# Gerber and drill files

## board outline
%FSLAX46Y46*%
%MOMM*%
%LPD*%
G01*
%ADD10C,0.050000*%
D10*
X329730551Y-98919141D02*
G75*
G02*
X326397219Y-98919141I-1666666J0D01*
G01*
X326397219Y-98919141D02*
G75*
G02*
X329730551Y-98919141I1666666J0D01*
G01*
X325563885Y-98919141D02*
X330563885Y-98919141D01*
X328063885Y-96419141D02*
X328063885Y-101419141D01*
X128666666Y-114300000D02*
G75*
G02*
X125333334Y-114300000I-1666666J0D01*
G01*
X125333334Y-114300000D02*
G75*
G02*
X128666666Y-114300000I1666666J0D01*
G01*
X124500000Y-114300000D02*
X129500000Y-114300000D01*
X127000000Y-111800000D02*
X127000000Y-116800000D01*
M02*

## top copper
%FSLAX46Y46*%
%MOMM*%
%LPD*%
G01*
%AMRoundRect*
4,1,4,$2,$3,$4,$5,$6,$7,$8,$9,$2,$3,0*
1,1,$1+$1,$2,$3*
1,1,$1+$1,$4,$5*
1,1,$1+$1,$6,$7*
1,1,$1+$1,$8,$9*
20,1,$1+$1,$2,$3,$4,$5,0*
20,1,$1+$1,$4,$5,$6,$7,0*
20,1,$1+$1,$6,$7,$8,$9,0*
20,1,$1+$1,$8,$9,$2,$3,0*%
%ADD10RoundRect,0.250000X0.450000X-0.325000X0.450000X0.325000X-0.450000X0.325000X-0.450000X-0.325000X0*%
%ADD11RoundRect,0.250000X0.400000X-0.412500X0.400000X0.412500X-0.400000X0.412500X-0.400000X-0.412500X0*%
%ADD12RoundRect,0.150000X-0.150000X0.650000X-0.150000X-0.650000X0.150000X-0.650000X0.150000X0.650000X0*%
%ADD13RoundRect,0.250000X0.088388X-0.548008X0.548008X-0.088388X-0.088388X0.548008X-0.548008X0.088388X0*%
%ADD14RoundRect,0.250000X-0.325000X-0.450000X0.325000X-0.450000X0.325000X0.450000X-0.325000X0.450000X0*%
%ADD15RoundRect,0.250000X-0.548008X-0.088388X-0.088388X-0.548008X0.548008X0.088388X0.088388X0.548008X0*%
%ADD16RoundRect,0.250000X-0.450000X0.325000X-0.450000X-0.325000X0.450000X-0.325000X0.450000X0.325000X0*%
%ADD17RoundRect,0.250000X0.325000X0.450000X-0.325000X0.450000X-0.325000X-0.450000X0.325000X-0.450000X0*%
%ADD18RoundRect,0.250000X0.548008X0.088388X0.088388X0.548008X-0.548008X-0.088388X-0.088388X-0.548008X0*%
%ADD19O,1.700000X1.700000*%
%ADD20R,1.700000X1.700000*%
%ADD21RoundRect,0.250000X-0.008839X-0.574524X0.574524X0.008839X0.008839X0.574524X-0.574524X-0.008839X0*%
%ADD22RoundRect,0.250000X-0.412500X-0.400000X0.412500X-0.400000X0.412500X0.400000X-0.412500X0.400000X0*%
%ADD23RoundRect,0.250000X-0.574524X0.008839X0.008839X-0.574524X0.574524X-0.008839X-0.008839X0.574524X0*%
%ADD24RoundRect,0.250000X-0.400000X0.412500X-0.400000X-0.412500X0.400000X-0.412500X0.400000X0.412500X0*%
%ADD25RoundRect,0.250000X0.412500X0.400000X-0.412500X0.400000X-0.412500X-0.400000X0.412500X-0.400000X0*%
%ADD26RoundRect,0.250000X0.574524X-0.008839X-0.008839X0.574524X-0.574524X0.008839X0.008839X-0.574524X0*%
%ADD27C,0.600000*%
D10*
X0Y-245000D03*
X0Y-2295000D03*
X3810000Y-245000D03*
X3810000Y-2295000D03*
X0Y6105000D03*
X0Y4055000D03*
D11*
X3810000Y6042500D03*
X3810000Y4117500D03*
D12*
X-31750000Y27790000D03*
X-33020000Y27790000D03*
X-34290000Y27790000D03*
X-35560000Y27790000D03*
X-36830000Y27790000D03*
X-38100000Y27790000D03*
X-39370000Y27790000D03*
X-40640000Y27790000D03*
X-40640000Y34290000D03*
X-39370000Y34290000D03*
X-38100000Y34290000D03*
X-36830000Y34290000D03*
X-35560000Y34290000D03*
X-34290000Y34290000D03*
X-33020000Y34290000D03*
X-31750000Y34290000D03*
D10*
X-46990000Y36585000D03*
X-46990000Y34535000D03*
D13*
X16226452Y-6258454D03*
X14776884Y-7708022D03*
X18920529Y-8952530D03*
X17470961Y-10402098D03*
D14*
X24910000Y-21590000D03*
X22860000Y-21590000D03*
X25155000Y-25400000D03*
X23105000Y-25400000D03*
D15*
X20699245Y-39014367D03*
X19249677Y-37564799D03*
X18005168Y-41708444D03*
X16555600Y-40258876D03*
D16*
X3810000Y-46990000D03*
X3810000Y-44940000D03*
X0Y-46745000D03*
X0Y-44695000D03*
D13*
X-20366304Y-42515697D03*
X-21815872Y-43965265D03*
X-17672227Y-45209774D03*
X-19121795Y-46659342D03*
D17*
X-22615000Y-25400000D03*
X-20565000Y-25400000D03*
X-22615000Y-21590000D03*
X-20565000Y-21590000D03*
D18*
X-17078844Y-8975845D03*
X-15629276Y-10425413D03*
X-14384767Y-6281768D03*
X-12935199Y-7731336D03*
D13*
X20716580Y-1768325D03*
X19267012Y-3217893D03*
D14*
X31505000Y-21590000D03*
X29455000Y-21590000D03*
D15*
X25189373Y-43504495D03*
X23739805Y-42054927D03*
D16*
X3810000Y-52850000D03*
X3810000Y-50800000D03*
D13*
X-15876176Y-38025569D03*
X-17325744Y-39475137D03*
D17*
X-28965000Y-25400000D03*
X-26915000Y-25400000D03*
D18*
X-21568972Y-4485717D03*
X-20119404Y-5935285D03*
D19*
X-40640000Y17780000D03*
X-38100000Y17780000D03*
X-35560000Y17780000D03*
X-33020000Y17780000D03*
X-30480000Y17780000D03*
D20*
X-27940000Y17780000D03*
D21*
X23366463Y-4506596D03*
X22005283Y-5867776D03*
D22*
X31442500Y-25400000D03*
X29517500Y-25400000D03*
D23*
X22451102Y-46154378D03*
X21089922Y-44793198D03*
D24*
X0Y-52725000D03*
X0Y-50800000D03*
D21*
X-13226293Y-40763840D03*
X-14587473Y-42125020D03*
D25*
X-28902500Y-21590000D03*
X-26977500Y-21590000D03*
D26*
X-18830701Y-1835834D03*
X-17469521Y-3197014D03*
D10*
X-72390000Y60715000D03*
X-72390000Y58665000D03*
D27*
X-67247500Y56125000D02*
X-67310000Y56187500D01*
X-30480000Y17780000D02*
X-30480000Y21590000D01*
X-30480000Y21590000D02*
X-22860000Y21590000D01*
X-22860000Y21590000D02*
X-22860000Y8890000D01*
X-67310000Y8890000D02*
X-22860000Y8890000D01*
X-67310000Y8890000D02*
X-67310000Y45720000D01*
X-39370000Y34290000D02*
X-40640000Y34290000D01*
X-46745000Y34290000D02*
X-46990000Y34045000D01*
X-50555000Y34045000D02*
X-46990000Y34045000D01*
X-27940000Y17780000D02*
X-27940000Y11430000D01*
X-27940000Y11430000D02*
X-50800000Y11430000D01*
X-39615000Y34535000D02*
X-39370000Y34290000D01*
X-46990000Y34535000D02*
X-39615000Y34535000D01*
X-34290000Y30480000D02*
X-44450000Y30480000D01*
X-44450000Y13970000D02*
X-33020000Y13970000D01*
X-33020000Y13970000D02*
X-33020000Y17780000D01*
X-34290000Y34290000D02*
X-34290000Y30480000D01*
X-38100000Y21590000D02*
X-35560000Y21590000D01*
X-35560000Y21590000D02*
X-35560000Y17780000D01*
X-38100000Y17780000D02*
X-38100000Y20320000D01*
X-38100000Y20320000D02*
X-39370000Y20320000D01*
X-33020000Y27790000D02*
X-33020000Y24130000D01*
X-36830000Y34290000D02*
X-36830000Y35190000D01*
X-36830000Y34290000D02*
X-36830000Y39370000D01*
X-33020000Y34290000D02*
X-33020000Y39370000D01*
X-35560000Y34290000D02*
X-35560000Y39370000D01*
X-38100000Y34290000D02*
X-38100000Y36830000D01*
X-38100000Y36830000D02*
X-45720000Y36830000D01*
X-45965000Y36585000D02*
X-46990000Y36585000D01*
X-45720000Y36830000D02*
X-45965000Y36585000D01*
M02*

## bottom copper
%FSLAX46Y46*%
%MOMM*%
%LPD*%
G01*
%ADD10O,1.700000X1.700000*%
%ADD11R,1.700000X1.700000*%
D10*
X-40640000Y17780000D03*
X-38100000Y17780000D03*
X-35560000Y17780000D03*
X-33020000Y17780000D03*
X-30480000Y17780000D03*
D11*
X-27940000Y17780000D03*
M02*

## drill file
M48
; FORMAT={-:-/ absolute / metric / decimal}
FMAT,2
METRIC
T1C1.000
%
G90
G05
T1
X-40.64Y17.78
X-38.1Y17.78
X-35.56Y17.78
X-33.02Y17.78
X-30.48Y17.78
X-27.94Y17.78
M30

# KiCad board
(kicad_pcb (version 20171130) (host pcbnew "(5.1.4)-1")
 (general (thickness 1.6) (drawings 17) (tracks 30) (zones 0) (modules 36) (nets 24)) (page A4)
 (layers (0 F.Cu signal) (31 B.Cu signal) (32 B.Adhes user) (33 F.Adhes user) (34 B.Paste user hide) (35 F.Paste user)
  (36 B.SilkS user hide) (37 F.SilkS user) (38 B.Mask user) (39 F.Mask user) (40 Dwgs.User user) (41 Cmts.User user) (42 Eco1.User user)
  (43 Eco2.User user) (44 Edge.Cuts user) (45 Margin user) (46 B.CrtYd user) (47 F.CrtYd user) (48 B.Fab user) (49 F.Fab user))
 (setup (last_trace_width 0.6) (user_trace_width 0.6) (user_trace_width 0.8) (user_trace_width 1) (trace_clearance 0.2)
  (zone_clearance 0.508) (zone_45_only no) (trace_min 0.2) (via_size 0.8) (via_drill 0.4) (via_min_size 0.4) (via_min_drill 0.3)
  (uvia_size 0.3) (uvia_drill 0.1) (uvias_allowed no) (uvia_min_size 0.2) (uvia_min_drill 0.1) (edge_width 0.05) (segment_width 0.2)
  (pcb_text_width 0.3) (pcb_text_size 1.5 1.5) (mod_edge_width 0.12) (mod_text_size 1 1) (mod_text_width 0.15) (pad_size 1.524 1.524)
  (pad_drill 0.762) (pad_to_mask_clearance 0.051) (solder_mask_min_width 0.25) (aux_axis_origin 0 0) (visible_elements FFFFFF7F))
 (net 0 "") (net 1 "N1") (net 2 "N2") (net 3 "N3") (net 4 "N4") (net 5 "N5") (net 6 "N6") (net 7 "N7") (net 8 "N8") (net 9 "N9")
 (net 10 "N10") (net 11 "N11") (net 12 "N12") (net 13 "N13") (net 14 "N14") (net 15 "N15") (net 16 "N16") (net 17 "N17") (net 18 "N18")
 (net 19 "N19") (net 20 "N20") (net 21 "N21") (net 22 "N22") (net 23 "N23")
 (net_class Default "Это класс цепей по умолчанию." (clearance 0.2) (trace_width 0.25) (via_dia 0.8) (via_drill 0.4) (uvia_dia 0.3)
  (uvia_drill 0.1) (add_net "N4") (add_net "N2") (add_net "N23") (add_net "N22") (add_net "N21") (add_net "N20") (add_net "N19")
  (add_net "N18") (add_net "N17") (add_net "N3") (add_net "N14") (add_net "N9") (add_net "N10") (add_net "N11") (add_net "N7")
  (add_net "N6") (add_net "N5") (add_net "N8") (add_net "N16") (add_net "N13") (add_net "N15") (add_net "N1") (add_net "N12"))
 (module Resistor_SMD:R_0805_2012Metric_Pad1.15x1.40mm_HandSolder (layer F.Cu) (at 0 1.27 90)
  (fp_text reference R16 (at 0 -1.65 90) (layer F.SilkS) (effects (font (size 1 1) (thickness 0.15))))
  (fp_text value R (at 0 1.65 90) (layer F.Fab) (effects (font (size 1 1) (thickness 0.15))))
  (pad 2 smd roundrect (at 1.025 0 90) (size 1.15 1.4) (layers F.Cu F.Paste F.Mask) (roundrect_rratio 0.217391) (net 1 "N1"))
  (pad 1 smd roundrect (at -1.025 0 90) (size 1.15 1.4) (layers F.Cu F.Paste F.Mask) (roundrect_rratio 0.217391) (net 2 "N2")))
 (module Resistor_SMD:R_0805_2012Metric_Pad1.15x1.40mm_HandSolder (layer F.Cu) (at 3.81 1.27 90)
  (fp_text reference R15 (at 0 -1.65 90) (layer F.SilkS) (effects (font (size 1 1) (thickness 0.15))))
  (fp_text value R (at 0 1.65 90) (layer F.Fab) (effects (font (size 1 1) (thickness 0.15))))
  (pad 2 smd roundrect (at 1.025 0 90) (size 1.15 1.4) (layers F.Cu F.Paste F.Mask) (roundrect_rratio 0.217391) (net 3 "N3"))
  (pad 1 smd roundrect (at -1.025 0 90) (size 1.15 1.4) (layers F.Cu F.Paste F.Mask) (roundrect_rratio 0.217391) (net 2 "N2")))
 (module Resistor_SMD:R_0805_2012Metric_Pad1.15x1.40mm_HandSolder (layer F.Cu) (at 0 -5.08 90)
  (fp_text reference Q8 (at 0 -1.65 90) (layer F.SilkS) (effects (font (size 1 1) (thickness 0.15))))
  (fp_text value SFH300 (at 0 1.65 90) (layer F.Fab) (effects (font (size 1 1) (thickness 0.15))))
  (pad 2 smd roundrect (at 1.025 0 90) (size 1.15 1.4) (layers F.Cu F.Paste F.Mask) (roundrect_rratio 0.217391) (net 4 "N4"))
  (pad 1 smd roundrect (at -1.025 0 90) (size 1.15 1.4) (layers F.Cu F.Paste F.Mask) (roundrect_rratio 0.217391) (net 1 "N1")))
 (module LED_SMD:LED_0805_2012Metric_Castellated (layer F.Cu) (at 3.81 -5.08 90)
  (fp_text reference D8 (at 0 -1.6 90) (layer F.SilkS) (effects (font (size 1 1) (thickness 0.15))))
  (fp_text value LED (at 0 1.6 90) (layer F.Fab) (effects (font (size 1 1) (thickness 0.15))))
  (pad 2 smd roundrect (at 0.9625 0 90) (size 1.325 1.3) (layers F.Cu F.Paste F.Mask) (roundrect_rratio 0.192308) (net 4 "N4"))
  (pad 1 smd roundrect (at -0.9625 0 90) (size 1.325 1.3) (layers F.Cu F.Paste F.Mask) (roundrect_rratio 0.192308) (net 3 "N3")))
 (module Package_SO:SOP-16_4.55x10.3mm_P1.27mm (layer F.Cu) (at -36.195 -31.04 270)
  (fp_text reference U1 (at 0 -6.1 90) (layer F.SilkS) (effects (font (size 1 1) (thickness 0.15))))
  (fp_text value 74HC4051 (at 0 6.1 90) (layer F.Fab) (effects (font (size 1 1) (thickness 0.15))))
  (pad 16 smd roundrect (at 3.25 -4.445 270) (size 1.6 0.6) (layers F.Cu F.Paste F.Mask) (roundrect_rratio 0.25) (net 4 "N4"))
  (pad 15 smd roundrect (at 3.25 -3.175 270) (size 1.6 0.6) (layers F.Cu F.Paste F.Mask) (roundrect_rratio 0.25) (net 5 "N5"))
  (pad 14 smd roundrect (at 3.25 -1.905 270) (size 1.6 0.6) (layers F.Cu F.Paste F.Mask) (roundrect_rratio 0.25) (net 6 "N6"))
  (pad 13 smd roundrect (at 3.25 -0.635 270) (size 1.6 0.6) (layers F.Cu F.Paste F.Mask) (roundrect_rratio 0.25) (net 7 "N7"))
  (pad 12 smd roundrect (at 3.25 0.635 270) (size 1.6 0.6) (layers F.Cu F.Paste F.Mask) (roundrect_rratio 0.25) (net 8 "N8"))
  (pad 11 smd roundrect (at 3.25 1.905 270) (size 1.6 0.6) (layers F.Cu F.Paste F.Mask) (roundrect_rratio 0.25) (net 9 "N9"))
  (pad 10 smd roundrect (at 3.25 3.175 270) (size 1.6 0.6) (layers F.Cu F.Paste F.Mask) (roundrect_rratio 0.25) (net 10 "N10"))
  (pad 9 smd roundrect (at 3.25 4.445 270) (size 1.6 0.6) (layers F.Cu F.Paste F.Mask) (roundrect_rratio 0.25) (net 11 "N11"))
  (pad 8 smd roundrect (at -3.25 4.445 270) (size 1.6 0.6) (layers F.Cu F.Paste F.Mask) (roundrect_rratio 0.25) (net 2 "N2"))
  (pad 7 smd roundrect (at -3.25 3.175 270) (size 1.6 0.6) (layers F.Cu F.Paste F.Mask) (roundrect_rratio 0.25) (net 2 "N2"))
  (pad 6 smd roundrect (at -3.25 1.905 270) (size 1.6 0.6) (layers F.Cu F.Paste F.Mask) (roundrect_rratio 0.25) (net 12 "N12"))
  (pad 5 smd roundrect (at -3.25 0.635 270) (size 1.6 0.6) (layers F.Cu F.Paste F.Mask) (roundrect_rratio 0.25) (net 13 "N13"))
  (pad 4 smd roundrect (at -3.25 -0.635 270) (size 1.6 0.6) (layers F.Cu F.Paste F.Mask) (roundrect_rratio 0.25) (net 1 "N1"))
  (pad 3 smd roundrect (at -3.25 -1.905 270) (size 1.6 0.6) (layers F.Cu F.Paste F.Mask) (roundrect_rratio 0.25) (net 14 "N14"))
  (pad 2 smd roundrect (at -3.25 -3.175 270) (size 1.6 0.6) (layers F.Cu F.Paste F.Mask) (roundrect_rratio 0.25) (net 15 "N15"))
  (pad 1 smd roundrect (at -3.25 -4.445 270) (size 1.6 0.6) (layers F.Cu F.Paste F.Mask) (roundrect_rratio 0.25) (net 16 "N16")))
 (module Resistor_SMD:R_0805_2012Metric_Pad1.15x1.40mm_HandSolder (layer F.Cu) (at -46.99 -35.56 90)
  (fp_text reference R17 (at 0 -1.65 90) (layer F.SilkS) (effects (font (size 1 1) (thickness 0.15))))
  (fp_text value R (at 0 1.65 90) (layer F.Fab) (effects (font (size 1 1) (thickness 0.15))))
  (pad 2 smd roundrect (at 1.025 0 90) (size 1.15 1.4) (layers F.Cu F.Paste F.Mask) (roundrect_rratio 0.217391) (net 12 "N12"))
  (pad 1 smd roundrect (at -1.025 0 90) (size 1.15 1.4) (layers F.Cu F.Paste F.Mask) (roundrect_rratio 0.217391) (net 2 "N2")))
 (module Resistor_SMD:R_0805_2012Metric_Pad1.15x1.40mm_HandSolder (layer F.Cu) (at 15.501668 6.983238 45)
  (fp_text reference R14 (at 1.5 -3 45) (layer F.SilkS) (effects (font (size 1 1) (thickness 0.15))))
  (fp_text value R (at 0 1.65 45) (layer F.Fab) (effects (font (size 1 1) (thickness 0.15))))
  (pad 2 smd roundrect (at 1.025 0 45) (size 1.15 1.4) (layers F.Cu F.Paste F.Mask) (roundrect_rratio 0.217391) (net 15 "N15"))
  (pad 1 smd roundrect (at -1.025 0 45) (size 1.15 1.4) (layers F.Cu F.Paste F.Mask) (roundrect_rratio 0.217391) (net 2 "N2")))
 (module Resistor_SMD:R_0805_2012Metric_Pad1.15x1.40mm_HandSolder (layer F.Cu) (at 18.195745 9.677314 45)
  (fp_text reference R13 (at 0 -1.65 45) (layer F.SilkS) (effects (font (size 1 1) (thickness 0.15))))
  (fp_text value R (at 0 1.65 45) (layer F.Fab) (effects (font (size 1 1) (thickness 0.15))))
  (pad 2 smd roundrect (at 1.025 0 45) (size 1.15 1.4) (layers F.Cu F.Paste F.Mask) (roundrect_rratio 0.217391) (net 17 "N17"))
  (pad 1 smd roundrect (at -1.025 0 45) (size 1.15 1.4) (layers F.Cu F.Paste F.Mask) (roundrect_rratio 0.217391) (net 2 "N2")))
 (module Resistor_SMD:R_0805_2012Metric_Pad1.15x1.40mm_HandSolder (layer F.Cu) (at 23.885 21.59)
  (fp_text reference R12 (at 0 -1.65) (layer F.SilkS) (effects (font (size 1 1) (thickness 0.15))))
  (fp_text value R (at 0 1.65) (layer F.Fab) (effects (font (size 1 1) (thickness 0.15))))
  (pad 2 smd roundrect (at 1.025 0) (size 1.15 1.4) (layers F.Cu F.Paste F.Mask) (roundrect_rratio 0.217391) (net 13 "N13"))
  (pad 1 smd roundrect (at -1.025 0) (size 1.15 1.4) (layers F.Cu F.Paste F.Mask) (roundrect_rratio 0.217391) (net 2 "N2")))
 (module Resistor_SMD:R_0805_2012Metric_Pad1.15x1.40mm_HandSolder (layer F.Cu) (at 24.13 25.4)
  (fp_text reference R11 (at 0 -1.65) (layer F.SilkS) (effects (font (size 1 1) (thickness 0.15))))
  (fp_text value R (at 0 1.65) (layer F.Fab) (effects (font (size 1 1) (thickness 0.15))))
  (pad 2 smd roundrect (at 1.025 0) (size 1.15 1.4) (layers F.Cu F.Paste F.Mask) (roundrect_rratio 0.217391) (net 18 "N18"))
  (pad 1 smd roundrect (at -1.025 0) (size 1.15 1.4) (layers F.Cu F.Paste F.Mask) (roundrect_rratio 0.217391) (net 2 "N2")))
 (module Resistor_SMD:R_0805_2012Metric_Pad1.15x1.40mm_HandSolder (layer F.Cu) (at 19.974461 38.289583 315)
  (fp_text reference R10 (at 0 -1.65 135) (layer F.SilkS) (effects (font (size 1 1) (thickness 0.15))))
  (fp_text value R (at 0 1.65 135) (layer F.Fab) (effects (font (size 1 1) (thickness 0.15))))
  (pad 2 smd roundrect (at 1.025 0 315) (size 1.15 1.4) (layers F.Cu F.Paste F.Mask) (roundrect_rratio 0.217391) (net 16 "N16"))
  (pad 1 smd roundrect (at -1.025 0 315) (size 1.15 1.4) (layers F.Cu F.Paste F.Mask) (roundrect_rratio 0.217391) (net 2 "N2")))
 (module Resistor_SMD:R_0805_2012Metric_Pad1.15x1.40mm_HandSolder (layer F.Cu) (at 17.280384 40.98366 315)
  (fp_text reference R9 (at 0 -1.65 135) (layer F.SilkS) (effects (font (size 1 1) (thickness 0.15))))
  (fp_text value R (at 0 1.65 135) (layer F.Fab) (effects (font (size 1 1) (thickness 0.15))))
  (pad 2 smd roundrect (at 1.025 0 315) (size 1.15 1.4) (layers F.Cu F.Paste F.Mask) (roundrect_rratio 0.217391) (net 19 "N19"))
  (pad 1 smd roundrect (at -1.025 0 315) (size 1.15 1.4) (layers F.Cu F.Paste F.Mask) (roundrect_rratio 0.217391) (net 2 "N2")))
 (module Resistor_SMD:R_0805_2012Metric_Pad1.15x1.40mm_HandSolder (layer F.Cu) (at 3.81 45.965 270)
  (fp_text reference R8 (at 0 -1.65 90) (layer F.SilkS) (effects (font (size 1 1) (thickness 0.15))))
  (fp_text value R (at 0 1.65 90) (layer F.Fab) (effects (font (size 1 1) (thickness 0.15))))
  (pad 2 smd roundrect (at 1.025 0 270) (size 1.15 1.4) (layers F.Cu F.Paste F.Mask) (roundrect_rratio 0.217391) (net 8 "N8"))
  (pad 1 smd roundrect (at -1.025 0 270) (size 1.15 1.4) (layers F.Cu F.Paste F.Mask) (roundrect_rratio 0.217391) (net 2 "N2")))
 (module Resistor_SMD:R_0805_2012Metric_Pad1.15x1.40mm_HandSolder (layer F.Cu) (at 0 45.72 270)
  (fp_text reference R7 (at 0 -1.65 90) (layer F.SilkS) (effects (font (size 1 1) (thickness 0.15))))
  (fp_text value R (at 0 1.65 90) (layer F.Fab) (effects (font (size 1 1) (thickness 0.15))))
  (pad 2 smd roundrect (at 1.025 0 270) (size 1.15 1.4) (layers F.Cu F.Paste F.Mask) (roundrect_rratio 0.217391) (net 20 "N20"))
  (pad 1 smd roundrect (at -1.025 0 270) (size 1.15 1.4) (layers F.Cu F.Paste F.Mask) (roundrect_rratio 0.217391) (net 2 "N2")))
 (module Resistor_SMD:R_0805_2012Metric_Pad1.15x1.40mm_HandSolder (layer F.Cu) (at -21.091088 43.240481 45)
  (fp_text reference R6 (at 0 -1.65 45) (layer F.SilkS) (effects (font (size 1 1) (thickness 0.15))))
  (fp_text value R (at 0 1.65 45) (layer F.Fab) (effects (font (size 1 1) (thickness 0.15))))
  (pad 2 smd roundrect (at 1.025 0 45) (size 1.15 1.4) (layers F.Cu F.Paste F.Mask) (roundrect_rratio 0.217391) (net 5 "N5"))
  (pad 1 smd roundrect (at -1.025 0 45) (size 1.15 1.4) (layers F.Cu F.Paste F.Mask) (roundrect_rratio 0.217391) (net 2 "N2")))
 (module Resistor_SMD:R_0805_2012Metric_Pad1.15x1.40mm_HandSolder (layer F.Cu) (at -18.397011 45.934558 45)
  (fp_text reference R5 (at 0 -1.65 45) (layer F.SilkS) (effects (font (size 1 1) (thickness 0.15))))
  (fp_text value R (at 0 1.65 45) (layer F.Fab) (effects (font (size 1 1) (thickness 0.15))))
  (pad 2 smd roundrect (at 1.025 0 45) (size 1.15 1.4) (layers F.Cu F.Paste F.Mask) (roundrect_rratio 0.217391) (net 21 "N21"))
  (pad 1 smd roundrect (at -1.025 0 45) (size 1.15 1.4) (layers F.Cu F.Paste F.Mask) (roundrect_rratio 0.217391) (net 2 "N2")))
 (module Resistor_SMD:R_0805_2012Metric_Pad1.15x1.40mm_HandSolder (layer F.Cu) (at -21.59 25.4 180)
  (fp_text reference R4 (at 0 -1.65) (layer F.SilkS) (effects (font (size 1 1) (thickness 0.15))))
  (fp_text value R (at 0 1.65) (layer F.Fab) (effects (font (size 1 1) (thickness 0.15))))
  (pad 2 smd roundrect (at 1.025 0 180) (size 1.15 1.4) (layers F.Cu F.Paste F.Mask) (roundrect_rratio 0.217391) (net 6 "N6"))
  (pad 1 smd roundrect (at -1.025 0 180) (size 1.15 1.4) (layers F.Cu F.Paste F.Mask) (roundrect_rratio 0.217391) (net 2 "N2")))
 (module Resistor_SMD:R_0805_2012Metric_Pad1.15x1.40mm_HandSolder (layer F.Cu) (at -21.59 21.59 180)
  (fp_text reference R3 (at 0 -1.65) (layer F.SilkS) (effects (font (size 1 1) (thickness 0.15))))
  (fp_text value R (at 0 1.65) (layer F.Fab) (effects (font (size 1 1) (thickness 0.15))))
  (pad 2 smd roundrect (at 1.025 0 180) (size 1.15 1.4) (layers F.Cu F.Paste F.Mask) (roundrect_rratio 0.217391) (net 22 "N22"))
  (pad 1 smd roundrect (at -1.025 0 180) (size 1.15 1.4) (layers F.Cu F.Paste F.Mask) (roundrect_rratio 0.217391) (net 2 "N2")))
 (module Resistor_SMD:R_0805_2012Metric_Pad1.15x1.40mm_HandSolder (layer F.Cu) (at -16.35406 9.700629 135)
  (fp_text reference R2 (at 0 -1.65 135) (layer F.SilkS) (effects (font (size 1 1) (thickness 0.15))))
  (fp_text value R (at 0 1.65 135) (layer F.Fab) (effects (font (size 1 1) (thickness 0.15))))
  (pad 2 smd roundrect (at 1.025 0 135) (size 1.15 1.4) (layers F.Cu F.Paste F.Mask) (roundrect_rratio 0.217391) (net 7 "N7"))
  (pad 1 smd roundrect (at -1.025 0 135) (size 1.15 1.4) (layers F.Cu F.Paste F.Mask) (roundrect_rratio 0.217391) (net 2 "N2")))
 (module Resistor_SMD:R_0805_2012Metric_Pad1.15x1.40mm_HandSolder (layer F.Cu) (at -13.659983 7.006552 135)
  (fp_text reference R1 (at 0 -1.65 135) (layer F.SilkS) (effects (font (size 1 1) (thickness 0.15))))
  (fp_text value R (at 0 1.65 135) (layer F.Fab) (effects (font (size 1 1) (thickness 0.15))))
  (pad 2 smd roundrect (at 1.025 0 135) (size 1.15 1.4) (layers F.Cu F.Paste F.Mask) (roundrect_rratio 0.217391) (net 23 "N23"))
  (pad 1 smd roundrect (at -1.025 0 135) (size 1.15 1.4) (layers F.Cu F.Paste F.Mask) (roundrect_rratio 0.217391) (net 2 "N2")))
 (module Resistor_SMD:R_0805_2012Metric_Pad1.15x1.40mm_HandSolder (layer F.Cu) (at 19.991796 2.493109 45)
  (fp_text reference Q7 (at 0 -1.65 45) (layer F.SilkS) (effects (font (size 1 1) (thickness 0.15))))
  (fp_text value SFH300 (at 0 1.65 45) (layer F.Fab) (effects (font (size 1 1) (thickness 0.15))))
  (pad 2 smd roundrect (at 1.025 0 45) (size 1.15 1.4) (layers F.Cu F.Paste F.Mask) (roundrect_rratio 0.217391) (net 4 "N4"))
  (pad 1 smd roundrect (at -1.025 0 45) (size 1.15 1.4) (layers F.Cu F.Paste F.Mask) (roundrect_rratio 0.217391) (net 15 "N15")))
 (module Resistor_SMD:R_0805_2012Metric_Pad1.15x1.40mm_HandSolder (layer F.Cu) (at 30.48 21.59)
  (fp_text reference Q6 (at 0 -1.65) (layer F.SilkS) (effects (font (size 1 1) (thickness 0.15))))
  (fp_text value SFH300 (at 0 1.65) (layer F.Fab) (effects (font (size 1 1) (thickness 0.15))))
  (pad 2 smd roundrect (at 1.025 0) (size 1.15 1.4) (layers F.Cu F.Paste F.Mask) (roundrect_rratio 0.217391) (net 4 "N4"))
  (pad 1 smd roundrect (at -1.025 0) (size 1.15 1.4) (layers F.Cu F.Paste F.Mask) (roundrect_rratio 0.217391) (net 13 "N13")))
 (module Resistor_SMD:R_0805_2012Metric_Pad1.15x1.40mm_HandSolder (layer F.Cu) (at 24.464589 42.779711 315)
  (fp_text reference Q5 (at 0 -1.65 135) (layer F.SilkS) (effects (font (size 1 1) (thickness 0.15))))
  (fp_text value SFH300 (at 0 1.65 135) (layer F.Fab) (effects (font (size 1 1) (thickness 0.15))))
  (pad 2 smd roundrect (at 1.025 0 315) (size 1.15 1.4) (layers F.Cu F.Paste F.Mask) (roundrect_rratio 0.217391) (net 4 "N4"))
  (pad 1 smd roundrect (at -1.025 0 315) (size 1.15 1.4) (layers F.Cu F.Paste F.Mask) (roundrect_rratio 0.217391) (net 16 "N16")))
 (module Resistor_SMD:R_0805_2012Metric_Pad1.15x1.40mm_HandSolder (layer F.Cu) (at 3.81 51.825 270)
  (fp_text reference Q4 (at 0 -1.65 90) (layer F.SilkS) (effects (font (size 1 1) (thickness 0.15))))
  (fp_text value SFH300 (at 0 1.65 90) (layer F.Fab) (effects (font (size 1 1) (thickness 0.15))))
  (pad 2 smd roundrect (at 1.025 0 270) (size 1.15 1.4) (layers F.Cu F.Paste F.Mask) (roundrect_rratio 0.217391) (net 4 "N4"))
  (pad 1 smd roundrect (at -1.025 0 270) (size 1.15 1.4) (layers F.Cu F.Paste F.Mask) (roundrect_rratio 0.217391) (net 8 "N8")))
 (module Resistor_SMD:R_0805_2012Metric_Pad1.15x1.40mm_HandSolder (layer F.Cu) (at -16.60096 38.750353 45)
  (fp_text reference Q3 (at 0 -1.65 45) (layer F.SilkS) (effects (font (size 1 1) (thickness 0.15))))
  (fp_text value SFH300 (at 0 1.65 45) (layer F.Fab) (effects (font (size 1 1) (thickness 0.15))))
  (pad 2 smd roundrect (at 1.025 0 45) (size 1.15 1.4) (layers F.Cu F.Paste F.Mask) (roundrect_rratio 0.217391) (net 4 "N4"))
  (pad 1 smd roundrect (at -1.025 0 45) (size 1.15 1.4) (layers F.Cu F.Paste F.Mask) (roundrect_rratio 0.217391) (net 5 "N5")))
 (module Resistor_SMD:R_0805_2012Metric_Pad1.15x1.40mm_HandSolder (layer F.Cu) (at -27.94 25.4 180)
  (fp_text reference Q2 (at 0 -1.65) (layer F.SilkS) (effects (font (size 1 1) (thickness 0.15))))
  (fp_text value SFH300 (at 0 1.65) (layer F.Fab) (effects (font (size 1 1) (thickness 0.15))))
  (pad 2 smd roundrect (at 1.025 0 180) (size 1.15 1.4) (layers F.Cu F.Paste F.Mask) (roundrect_rratio 0.217391) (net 4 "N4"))
  (pad 1 smd roundrect (at -1.025 0 180) (size 1.15 1.4) (layers F.Cu F.Paste F.Mask) (roundrect_rratio 0.217391) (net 6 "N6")))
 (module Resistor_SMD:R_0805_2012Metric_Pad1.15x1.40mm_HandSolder (layer F.Cu) (at -20.844188 5.210501 135)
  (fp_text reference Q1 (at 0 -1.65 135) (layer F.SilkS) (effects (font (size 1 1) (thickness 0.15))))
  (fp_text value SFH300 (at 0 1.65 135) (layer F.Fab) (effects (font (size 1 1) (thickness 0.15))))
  (pad 2 smd roundrect (at 1.025 0 135) (size 1.15 1.4) (layers F.Cu F.Paste F.Mask) (roundrect_rratio 0.217391) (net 4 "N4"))
  (pad 1 smd roundrect (at -1.025 0 135) (size 1.15 1.4) (layers F.Cu F.Paste F.Mask) (roundrect_rratio 0.217391) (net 7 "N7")))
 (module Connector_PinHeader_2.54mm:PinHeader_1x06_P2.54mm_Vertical (layer F.Cu) (at -27.94 -17.78 270)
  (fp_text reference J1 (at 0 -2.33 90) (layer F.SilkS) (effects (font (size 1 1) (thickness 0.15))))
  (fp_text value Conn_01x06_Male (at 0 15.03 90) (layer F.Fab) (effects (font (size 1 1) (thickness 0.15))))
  (pad 6 thru_hole oval (at 0 12.7 270) (size 1.7 1.7) (drill 1) (layers *.Cu *.Mask) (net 11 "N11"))
  (pad 5 thru_hole oval (at 0 10.16 270) (size 1.7 1.7) (drill 1) (layers *.Cu *.Mask) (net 10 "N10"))
  (pad 4 thru_hole oval (at 0 7.62 270) (size 1.7 1.7) (drill 1) (layers *.Cu *.Mask) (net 9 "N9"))
  (pad 3 thru_hole oval (at 0 5.08 270) (size 1.7 1.7) (drill 1) (layers *.Cu *.Mask) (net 14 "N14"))
  (pad 2 thru_hole oval (at 0 2.54 270) (size 1.7 1.7) (drill 1) (layers *.Cu *.Mask) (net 4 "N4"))
  (pad 1 thru_hole rect (at 0 0 270) (size 1.7 1.7) (drill 1) (layers *.Cu *.Mask) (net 2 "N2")))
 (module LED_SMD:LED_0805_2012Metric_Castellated (layer F.Cu) (at 22.685873 5.187186 45)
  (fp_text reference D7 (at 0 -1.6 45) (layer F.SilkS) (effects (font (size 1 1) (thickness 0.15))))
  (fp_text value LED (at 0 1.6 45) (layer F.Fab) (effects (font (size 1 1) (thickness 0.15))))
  (pad 2 smd roundrect (at 0.9625 0 45) (size 1.325 1.3) (layers F.Cu F.Paste F.Mask) (roundrect_rratio 0.192308) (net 4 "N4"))
  (pad 1 smd roundrect (at -0.9625 0 45) (size 1.325 1.3) (layers F.Cu F.Paste F.Mask) (roundrect_rratio 0.192308) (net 17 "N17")))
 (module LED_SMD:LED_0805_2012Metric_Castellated (layer F.Cu) (at 30.48 25.4)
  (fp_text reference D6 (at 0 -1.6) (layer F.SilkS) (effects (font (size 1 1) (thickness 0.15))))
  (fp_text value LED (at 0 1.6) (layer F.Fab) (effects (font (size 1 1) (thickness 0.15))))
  (pad 2 smd roundrect (at 0.9625 0) (size 1.325 1.3) (layers F.Cu F.Paste F.Mask) (roundrect_rratio 0.192308) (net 4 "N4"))
  (pad 1 smd roundrect (at -0.9625 0) (size 1.325 1.3) (layers F.Cu F.Paste F.Mask) (roundrect_rratio 0.192308) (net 18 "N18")))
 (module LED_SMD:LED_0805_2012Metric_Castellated (layer F.Cu) (at 21.770512 45.473788 315)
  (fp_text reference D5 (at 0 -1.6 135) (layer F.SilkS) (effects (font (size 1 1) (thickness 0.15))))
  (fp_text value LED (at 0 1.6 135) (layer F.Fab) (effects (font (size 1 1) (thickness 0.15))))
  (pad 2 smd roundrect (at 0.9625 0 315) (size 1.325 1.3) (layers F.Cu F.Paste F.Mask) (roundrect_rratio 0.192308) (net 4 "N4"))
  (pad 1 smd roundrect (at -0.9625 0 315) (size 1.325 1.3) (layers F.Cu F.Paste F.Mask) (roundrect_rratio 0.192308) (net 19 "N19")))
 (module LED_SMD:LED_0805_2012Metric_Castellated (layer F.Cu) (at 0 51.7625 270)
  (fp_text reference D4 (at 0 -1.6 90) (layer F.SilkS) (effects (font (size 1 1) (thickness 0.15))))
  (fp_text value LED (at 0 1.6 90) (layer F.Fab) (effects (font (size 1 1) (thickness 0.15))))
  (pad 2 smd roundrect (at 0.9625 0 270) (size 1.325 1.3) (layers F.Cu F.Paste F.Mask) (roundrect_rratio 0.192308) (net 4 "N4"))
  (pad 1 smd roundrect (at -0.9625 0 270) (size 1.325 1.3) (layers F.Cu F.Paste F.Mask) (roundrect_rratio 0.192308) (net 20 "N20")))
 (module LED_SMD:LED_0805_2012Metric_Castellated (layer F.Cu) (at -13.906883 41.44443 45)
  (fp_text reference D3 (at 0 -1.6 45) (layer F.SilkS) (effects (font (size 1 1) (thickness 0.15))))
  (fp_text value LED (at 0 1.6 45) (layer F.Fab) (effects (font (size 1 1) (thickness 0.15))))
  (pad 2 smd roundrect (at 0.9625 0 45) (size 1.325 1.3) (layers F.Cu F.Paste F.Mask) (roundrect_rratio 0.192308) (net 4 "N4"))
  (pad 1 smd roundrect (at -0.9625 0 45) (size 1.325 1.3) (layers F.Cu F.Paste F.Mask) (roundrect_rratio 0.192308) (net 21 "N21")))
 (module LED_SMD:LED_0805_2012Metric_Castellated (layer F.Cu) (at -27.94 21.59 180)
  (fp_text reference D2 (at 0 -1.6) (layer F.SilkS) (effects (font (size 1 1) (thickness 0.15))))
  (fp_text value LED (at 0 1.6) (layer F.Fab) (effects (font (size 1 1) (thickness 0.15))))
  (pad 2 smd roundrect (at 0.9625 0 180) (size 1.325 1.3) (layers F.Cu F.Paste F.Mask) (roundrect_rratio 0.192308) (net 4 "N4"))
  (pad 1 smd roundrect (at -0.9625 0 180) (size 1.325 1.3) (layers F.Cu F.Paste F.Mask) (roundrect_rratio 0.192308) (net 22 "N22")))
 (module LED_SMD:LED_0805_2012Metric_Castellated (layer F.Cu) (at -18.150111 2.516424 135)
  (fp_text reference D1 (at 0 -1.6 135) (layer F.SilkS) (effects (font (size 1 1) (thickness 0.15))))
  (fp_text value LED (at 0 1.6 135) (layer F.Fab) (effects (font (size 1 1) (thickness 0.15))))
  (pad 2 smd roundrect (at 0.9625 0 135) (size 1.325 1.3) (layers F.Cu F.Paste F.Mask) (roundrect_rratio 0.192308) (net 4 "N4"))
  (pad 1 smd roundrect (at -0.9625 0 135) (size 1.325 1.3) (layers F.Cu F.Paste F.Mask) (roundrect_rratio 0.192308) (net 23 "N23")))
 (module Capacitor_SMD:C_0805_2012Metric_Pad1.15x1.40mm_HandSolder (layer F.Cu) (at -72.39 -59.69 90)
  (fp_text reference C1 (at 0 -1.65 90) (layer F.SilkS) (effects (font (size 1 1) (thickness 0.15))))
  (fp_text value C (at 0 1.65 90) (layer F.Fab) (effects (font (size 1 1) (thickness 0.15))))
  (pad 2 smd roundrect (at 1.025 0 90) (size 1.15 1.4) (layers F.Cu F.Paste F.Mask) (roundrect_rratio 0.217391) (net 2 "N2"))
  (pad 1 smd roundrect (at -1.025 0 90) (size 1.15 1.4) (layers F.Cu F.Paste F.Mask) (roundrect_rratio 0.217391) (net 4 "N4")))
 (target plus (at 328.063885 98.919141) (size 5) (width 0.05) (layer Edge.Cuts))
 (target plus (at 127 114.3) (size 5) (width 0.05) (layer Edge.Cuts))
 (segment (start -67.2475 -56.125) (end -67.31 -56.1875) (width 0.6) (layer F.Cu) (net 4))
 (segment (start -30.48 -17.78) (end -30.48 -21.59) (width 0.6) (layer F.Cu) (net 4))
 (segment (start -30.48 -21.59) (end -22.86 -21.59) (width 0.6) (layer F.Cu) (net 4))
 (segment (start -22.86 -21.59) (end -22.86 -8.89) (width 0.6) (layer F.Cu) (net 4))
 (segment (start -67.31 -8.89) (end -22.86 -8.89) (width 0.6) (layer F.Cu) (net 4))
 (segment (start -67.31 -8.89) (end -67.31 -45.72) (width 0.6) (layer F.Cu) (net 4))
 (segment (start -39.37 -34.29) (end -40.64 -34.29) (width 0.6) (layer F.Cu) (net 2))
 (segment (start -46.745 -34.29) (end -46.99 -34.045) (width 0.6) (layer F.Cu) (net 2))
 (segment (start -50.555 -34.045) (end -46.99 -34.045) (width 0.6) (layer F.Cu) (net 2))
 (segment (start -27.94 -17.78) (end -27.94 -11.43) (width 0.6) (layer F.Cu) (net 2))
 (segment (start -27.94 -11.43) (end -50.8 -11.43) (width 0.6) (layer F.Cu) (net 2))
 (segment (start -39.615 -34.535) (end -39.37 -34.29) (width 0.6) (layer F.Cu) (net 2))
 (segment (start -46.99 -34.535) (end -39.615 -34.535) (width 0.6) (layer F.Cu) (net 2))
 (segment (start -34.29 -30.48) (end -44.45 -30.48) (width 0.6) (layer F.Cu) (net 14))
 (segment (start -44.45 -13.97) (end -33.02 -13.97) (width 0.6) (layer F.Cu) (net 14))
 (segment (start -33.02 -13.97) (end -33.02 -17.78) (width 0.6) (layer F.Cu) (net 14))
 (segment (start -34.29 -34.29) (end -34.29 -30.48) (width 0.6) (layer F.Cu) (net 14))
 (segment (start -38.1 -21.59) (end -35.56 -21.59) (width 0.6) (layer F.Cu) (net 9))
 (segment (start -35.56 -21.59) (end -35.56 -17.78) (width 0.6) (layer F.Cu) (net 9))
 (segment (start -38.1 -17.78) (end -38.1 -20.32) (width 0.6) (layer F.Cu) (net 10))
 (segment (start -38.1 -20.32) (end -39.37 -20.32) (width 0.6) (layer F.Cu) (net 10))
 (segment (start -33.02 -27.79) (end -33.02 -24.13) (width 0.6) (layer F.Cu) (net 5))
 (segment (start -36.83 -34.29) (end -36.83 -35.19) (width 0.6) (layer F.Cu) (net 13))
 (segment (start -36.83 -34.29) (end -36.83 -39.37) (width 0.6) (layer F.Cu) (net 13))
 (segment (start -33.02 -34.29) (end -33.02 -39.37) (width 0.6) (layer F.Cu) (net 15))
 (segment (start -35.56 -34.29) (end -35.56 -39.37) (width 0.6) (layer F.Cu) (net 1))
 (segment (start -38.1 -34.29) (end -38.1 -36.83) (width 0.6) (layer F.Cu) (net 12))
 (segment (start -38.1 -36.83) (end -45.72 -36.83) (width 0.6) (layer F.Cu) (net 12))
 (segment (start -45.965 -36.585) (end -46.99 -36.585) (width 0.6) (layer F.Cu) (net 12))
 (segment (start -45.72 -36.83) (end -45.965 -36.585) (width 0.6) (layer F.Cu) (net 12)))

